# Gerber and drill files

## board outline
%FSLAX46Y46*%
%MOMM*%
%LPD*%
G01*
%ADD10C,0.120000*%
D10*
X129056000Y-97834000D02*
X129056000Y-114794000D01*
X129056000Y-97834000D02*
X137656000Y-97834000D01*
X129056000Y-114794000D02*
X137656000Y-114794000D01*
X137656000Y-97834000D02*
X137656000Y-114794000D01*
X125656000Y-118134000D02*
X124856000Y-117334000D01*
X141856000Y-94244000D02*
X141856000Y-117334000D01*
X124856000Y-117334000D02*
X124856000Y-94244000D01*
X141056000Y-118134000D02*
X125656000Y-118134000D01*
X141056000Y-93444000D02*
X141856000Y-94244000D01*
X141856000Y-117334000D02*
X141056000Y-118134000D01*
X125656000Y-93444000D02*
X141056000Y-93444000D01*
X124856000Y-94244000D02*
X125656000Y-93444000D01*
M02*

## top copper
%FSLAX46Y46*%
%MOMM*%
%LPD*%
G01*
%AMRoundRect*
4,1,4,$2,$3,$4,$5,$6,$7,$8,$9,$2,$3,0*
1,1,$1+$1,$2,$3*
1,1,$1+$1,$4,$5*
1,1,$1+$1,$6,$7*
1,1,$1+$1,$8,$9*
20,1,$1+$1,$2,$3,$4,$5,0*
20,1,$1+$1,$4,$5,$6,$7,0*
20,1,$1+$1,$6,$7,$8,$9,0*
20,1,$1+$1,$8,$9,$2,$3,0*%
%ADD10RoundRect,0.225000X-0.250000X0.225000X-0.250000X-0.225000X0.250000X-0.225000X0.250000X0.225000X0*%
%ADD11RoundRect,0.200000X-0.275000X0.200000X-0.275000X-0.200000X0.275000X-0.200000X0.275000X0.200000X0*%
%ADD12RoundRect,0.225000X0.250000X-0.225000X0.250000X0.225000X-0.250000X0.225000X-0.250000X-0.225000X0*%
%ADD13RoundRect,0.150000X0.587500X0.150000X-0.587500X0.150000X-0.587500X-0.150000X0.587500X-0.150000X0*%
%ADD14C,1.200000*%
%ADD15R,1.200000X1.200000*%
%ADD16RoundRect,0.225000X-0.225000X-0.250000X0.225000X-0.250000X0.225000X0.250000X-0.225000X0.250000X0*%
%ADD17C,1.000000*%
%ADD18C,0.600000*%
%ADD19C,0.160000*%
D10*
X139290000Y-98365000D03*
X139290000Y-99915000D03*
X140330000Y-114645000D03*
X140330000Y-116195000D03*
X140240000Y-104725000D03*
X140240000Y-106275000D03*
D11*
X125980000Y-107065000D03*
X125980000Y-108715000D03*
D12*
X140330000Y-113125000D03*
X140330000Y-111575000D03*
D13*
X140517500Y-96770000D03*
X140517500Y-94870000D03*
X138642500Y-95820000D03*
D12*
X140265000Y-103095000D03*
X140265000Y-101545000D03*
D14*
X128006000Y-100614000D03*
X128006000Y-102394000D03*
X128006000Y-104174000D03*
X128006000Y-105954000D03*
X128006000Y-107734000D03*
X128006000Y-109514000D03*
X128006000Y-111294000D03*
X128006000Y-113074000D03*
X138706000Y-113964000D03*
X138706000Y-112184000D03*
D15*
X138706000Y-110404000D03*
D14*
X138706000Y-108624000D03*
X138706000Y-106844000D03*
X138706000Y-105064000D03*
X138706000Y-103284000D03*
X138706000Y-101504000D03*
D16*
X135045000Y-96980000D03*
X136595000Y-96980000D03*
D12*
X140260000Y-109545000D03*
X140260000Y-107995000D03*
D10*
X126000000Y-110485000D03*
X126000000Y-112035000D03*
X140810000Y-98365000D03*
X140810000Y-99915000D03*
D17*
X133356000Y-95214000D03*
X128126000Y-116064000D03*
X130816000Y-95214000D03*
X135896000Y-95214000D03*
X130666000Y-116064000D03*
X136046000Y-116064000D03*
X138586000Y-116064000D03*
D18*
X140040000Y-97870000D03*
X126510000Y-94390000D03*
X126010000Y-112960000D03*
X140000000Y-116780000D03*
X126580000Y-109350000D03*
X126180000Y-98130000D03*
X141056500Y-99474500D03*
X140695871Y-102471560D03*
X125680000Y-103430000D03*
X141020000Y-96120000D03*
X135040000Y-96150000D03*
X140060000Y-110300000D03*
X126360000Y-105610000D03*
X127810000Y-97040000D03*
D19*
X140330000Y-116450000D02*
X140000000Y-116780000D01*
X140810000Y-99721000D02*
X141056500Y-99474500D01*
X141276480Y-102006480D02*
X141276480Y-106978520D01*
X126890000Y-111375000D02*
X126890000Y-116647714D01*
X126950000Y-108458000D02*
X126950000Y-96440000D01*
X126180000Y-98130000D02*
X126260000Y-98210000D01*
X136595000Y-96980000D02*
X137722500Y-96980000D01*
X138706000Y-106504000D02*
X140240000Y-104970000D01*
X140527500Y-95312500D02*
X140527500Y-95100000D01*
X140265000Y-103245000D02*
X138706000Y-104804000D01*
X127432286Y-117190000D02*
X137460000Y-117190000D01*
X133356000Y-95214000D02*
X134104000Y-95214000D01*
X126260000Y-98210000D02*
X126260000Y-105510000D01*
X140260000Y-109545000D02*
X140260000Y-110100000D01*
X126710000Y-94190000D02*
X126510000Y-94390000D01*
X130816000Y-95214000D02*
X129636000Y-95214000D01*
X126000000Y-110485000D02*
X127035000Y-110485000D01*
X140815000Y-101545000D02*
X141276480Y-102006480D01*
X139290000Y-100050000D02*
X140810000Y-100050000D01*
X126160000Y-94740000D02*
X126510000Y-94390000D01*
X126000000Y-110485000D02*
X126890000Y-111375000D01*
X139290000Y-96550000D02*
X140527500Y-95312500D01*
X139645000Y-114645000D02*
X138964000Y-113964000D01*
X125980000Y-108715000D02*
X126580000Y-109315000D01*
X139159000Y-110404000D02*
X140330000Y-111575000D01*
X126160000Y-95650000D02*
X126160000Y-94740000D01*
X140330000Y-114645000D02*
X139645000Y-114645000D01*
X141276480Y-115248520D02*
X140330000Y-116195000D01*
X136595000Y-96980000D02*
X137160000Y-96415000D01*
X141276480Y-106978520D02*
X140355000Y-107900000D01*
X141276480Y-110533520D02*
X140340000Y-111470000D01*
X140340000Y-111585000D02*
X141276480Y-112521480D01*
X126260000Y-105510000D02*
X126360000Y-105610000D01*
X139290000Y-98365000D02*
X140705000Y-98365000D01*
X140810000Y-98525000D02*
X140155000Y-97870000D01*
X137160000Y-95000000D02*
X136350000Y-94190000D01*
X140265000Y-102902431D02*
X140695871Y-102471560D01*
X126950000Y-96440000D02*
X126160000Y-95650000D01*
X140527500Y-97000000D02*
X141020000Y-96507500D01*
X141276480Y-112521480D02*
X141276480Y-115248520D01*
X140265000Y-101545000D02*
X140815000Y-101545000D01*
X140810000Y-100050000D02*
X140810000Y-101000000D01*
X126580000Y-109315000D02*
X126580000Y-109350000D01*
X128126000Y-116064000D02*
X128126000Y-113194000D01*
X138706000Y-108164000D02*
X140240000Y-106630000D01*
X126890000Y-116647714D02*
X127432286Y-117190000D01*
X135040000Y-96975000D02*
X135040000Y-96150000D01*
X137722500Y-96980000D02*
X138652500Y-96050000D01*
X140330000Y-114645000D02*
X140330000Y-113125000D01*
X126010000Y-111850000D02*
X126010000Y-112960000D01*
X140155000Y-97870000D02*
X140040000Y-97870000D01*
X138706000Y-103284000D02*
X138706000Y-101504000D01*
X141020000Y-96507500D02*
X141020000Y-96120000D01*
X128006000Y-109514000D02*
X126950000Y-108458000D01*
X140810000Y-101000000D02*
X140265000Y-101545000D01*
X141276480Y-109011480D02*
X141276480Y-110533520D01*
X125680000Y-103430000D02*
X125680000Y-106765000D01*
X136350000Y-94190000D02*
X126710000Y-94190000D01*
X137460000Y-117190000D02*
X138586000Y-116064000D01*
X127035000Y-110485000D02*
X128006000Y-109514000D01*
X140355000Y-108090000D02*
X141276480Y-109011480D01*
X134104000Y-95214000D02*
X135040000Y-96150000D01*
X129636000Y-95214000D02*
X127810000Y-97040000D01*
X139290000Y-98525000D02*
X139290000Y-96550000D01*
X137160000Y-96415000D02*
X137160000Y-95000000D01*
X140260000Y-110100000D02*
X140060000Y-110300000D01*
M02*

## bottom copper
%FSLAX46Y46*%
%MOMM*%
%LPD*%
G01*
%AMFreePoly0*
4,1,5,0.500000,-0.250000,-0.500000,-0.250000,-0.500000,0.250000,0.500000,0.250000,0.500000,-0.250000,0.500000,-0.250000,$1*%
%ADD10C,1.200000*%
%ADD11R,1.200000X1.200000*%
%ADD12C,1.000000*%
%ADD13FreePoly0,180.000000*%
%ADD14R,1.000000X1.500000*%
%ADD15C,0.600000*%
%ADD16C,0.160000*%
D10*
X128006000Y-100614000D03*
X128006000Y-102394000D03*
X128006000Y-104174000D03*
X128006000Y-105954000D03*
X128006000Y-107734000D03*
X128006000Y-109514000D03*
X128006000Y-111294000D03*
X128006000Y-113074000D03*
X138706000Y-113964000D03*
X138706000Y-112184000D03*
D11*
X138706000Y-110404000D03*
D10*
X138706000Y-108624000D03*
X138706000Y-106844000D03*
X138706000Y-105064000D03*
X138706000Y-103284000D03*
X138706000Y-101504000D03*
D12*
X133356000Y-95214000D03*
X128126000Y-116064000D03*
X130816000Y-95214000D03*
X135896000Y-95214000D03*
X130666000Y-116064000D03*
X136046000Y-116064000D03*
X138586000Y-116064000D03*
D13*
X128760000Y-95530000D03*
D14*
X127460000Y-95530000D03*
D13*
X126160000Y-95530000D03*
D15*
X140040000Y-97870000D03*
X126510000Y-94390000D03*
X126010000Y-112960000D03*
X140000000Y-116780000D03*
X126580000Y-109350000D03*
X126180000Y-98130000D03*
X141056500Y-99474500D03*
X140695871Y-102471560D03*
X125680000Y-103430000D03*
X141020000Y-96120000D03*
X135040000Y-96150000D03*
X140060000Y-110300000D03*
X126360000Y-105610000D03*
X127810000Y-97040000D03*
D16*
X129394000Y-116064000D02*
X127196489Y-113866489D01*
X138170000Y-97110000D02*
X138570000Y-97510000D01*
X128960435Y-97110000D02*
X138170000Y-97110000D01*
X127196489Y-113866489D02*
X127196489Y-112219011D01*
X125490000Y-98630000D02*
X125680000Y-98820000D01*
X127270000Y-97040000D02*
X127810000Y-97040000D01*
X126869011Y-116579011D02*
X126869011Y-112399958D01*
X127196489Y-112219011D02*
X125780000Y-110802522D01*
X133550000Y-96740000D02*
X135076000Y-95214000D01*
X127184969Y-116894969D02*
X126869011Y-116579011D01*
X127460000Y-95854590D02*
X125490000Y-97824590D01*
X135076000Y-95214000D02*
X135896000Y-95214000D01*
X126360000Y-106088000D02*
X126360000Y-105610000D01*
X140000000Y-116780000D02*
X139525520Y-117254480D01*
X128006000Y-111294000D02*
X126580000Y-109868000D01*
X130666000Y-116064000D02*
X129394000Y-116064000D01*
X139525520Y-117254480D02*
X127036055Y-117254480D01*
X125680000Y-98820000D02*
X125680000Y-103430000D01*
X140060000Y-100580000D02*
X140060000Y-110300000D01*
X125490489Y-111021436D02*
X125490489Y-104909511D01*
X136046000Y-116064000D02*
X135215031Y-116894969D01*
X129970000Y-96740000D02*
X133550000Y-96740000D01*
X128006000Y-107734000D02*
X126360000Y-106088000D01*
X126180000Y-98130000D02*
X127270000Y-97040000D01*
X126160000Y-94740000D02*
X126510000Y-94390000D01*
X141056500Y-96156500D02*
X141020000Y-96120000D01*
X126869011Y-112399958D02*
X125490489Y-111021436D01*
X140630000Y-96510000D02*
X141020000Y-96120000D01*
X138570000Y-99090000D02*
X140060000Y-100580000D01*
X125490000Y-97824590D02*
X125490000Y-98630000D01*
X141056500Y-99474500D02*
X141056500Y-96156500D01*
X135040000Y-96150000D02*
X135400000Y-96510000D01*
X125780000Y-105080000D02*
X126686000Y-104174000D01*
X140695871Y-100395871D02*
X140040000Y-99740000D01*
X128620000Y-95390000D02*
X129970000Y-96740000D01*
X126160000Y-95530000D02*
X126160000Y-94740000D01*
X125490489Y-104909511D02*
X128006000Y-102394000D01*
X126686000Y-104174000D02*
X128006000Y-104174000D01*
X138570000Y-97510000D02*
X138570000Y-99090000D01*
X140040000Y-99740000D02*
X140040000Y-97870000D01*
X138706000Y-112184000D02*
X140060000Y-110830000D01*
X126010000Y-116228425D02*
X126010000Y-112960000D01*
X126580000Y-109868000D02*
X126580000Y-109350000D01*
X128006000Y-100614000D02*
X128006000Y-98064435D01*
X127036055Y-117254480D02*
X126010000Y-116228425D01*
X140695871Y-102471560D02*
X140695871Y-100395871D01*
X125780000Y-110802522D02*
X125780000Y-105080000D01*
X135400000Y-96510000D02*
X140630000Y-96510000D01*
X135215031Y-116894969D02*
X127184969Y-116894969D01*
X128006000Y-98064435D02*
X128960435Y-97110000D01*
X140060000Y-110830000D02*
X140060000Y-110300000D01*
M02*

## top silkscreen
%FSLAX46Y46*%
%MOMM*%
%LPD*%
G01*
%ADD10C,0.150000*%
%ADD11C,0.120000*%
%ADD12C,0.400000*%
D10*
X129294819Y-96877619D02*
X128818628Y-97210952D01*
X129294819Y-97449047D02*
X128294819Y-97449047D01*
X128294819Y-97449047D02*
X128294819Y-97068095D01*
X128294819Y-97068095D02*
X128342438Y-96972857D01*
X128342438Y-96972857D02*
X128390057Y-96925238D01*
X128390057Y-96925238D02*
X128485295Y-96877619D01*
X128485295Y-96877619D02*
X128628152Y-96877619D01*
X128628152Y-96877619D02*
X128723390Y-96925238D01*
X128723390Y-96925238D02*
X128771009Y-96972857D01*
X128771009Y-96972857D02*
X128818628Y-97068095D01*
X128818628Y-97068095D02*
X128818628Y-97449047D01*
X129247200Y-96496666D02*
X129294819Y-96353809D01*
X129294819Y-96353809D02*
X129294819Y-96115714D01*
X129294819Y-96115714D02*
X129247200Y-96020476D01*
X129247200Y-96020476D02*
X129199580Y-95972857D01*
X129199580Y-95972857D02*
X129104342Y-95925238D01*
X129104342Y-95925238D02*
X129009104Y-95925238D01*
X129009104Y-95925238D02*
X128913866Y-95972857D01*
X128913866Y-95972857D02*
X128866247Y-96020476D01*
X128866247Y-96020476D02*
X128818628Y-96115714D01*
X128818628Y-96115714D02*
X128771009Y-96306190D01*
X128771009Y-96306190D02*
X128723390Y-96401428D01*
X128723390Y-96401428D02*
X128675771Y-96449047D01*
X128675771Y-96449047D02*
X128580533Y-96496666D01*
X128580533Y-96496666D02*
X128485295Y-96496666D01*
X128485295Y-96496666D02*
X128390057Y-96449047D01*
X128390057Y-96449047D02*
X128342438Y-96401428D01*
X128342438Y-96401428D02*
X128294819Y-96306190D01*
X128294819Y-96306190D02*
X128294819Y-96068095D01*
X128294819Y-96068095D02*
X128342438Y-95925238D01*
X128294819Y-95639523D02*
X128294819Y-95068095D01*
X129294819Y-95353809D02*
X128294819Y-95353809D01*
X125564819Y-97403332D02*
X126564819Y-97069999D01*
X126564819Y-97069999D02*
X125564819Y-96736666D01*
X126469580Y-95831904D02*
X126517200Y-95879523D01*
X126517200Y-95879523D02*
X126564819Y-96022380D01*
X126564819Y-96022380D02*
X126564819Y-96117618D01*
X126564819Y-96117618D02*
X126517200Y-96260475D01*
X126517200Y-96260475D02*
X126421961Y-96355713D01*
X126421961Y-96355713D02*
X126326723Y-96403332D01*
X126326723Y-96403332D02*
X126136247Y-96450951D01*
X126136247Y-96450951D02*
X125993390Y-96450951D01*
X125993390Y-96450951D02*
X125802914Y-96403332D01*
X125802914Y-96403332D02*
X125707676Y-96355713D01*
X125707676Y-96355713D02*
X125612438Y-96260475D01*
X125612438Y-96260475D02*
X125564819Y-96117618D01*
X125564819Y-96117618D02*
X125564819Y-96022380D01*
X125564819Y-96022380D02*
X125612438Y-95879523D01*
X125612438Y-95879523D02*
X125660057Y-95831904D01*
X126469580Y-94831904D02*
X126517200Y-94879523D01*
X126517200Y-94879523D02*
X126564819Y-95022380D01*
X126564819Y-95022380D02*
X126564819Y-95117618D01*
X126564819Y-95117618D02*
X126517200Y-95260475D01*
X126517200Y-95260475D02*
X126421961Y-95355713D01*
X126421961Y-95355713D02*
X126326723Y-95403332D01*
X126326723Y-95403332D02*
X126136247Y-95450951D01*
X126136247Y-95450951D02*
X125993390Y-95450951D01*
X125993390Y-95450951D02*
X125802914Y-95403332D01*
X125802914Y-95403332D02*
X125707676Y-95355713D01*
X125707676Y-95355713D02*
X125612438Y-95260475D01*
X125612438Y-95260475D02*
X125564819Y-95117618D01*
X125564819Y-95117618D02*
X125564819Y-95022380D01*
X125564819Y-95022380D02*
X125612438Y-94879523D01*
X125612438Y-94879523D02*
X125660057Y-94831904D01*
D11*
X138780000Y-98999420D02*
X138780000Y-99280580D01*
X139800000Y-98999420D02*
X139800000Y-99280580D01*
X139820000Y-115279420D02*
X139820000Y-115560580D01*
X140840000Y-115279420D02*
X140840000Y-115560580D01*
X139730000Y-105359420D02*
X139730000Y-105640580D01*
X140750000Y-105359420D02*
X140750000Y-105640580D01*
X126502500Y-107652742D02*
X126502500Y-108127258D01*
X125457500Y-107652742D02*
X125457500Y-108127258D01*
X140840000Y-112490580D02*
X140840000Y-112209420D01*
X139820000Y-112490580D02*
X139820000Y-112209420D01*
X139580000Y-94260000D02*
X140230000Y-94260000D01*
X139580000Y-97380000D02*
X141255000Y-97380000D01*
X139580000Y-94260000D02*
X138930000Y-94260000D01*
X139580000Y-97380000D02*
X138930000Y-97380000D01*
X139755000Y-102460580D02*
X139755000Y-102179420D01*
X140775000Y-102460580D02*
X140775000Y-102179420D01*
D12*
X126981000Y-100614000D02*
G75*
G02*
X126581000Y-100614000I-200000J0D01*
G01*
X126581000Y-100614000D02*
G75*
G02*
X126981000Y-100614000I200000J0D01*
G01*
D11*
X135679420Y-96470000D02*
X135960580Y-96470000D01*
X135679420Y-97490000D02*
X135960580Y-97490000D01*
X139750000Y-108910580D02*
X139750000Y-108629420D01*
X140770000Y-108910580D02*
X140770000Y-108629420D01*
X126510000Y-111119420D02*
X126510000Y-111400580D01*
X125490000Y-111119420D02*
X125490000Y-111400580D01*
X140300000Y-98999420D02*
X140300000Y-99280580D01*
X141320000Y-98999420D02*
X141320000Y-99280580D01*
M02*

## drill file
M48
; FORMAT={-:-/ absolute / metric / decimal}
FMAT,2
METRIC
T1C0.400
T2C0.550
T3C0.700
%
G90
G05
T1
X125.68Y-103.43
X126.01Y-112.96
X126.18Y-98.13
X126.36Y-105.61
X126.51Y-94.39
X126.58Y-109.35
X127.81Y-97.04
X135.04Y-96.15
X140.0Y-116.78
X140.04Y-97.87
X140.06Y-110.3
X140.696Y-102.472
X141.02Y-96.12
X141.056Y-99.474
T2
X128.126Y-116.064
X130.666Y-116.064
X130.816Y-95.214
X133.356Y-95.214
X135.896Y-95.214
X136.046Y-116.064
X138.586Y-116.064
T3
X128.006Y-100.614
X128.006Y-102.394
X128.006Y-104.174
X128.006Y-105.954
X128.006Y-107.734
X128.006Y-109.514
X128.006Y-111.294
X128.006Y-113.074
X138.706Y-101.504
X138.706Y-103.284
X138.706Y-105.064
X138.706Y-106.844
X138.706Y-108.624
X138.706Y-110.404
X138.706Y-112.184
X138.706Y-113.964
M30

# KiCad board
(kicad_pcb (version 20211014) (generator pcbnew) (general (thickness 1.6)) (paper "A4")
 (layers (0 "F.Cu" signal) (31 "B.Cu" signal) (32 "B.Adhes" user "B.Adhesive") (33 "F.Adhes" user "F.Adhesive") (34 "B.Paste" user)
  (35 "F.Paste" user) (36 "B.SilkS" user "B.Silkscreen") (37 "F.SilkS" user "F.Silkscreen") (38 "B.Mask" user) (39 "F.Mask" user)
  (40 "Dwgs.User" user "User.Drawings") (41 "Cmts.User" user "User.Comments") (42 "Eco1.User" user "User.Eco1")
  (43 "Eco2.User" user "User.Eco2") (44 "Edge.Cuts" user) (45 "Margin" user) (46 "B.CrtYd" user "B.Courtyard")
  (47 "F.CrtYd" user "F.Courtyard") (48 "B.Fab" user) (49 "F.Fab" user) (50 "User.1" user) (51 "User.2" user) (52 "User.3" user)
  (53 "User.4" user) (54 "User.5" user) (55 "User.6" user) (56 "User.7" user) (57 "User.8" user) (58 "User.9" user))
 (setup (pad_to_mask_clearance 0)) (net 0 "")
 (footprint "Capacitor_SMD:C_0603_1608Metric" (layer "F.Cu") (at 139.29 99.14 -90)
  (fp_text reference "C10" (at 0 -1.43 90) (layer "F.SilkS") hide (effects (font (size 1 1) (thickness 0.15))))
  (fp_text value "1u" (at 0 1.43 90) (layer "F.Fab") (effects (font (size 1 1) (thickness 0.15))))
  (fp_line (start -0.14058 0.51) (end 0.14058 0.51) (layer "F.SilkS") (width 0.12))
  (fp_line (start -0.14058 -0.51) (end 0.14058 -0.51) (layer "F.SilkS") (width 0.12))
  (pad "1" smd roundrect (at -0.775 0 270) (size 0.9 0.95) (layers "F.Cu" "F.Paste" "F.Mask") (roundrect_rratio 0.25))
  (pad "2" smd roundrect (at 0.775 0 270) (size 0.9 0.95) (layers "F.Cu" "F.Paste" "F.Mask") (roundrect_rratio 0.25)))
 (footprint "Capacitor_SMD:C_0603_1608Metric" (layer "F.Cu") (at 140.33 115.42 -90)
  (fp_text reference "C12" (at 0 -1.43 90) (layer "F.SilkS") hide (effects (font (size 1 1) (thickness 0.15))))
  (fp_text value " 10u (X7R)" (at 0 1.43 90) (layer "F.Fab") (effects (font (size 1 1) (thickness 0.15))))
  (fp_line (start -0.14058 0.51) (end 0.14058 0.51) (layer "F.SilkS") (width 0.12))
  (fp_line (start -0.14058 -0.51) (end 0.14058 -0.51) (layer "F.SilkS") (width 0.12))
  (pad "1" smd roundrect (at -0.775 0 270) (size 0.9 0.95) (layers "F.Cu" "F.Paste" "F.Mask") (roundrect_rratio 0.25))
  (pad "2" smd roundrect (at 0.775 0 270) (size 0.9 0.95) (layers "F.Cu" "F.Paste" "F.Mask") (roundrect_rratio 0.25)))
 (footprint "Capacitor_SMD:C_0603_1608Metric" (layer "F.Cu") (at 140.24 105.5 -90)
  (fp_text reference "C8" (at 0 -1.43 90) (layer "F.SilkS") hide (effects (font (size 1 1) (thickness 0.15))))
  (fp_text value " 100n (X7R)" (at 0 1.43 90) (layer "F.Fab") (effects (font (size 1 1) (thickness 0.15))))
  (fp_line (start -0.14058 0.51) (end 0.14058 0.51) (layer "F.SilkS") (width 0.12))
  (fp_line (start -0.14058 -0.51) (end 0.14058 -0.51) (layer "F.SilkS") (width 0.12))
  (pad "1" smd roundrect (at -0.775 0 270) (size 0.9 0.95) (layers "F.Cu" "F.Paste" "F.Mask") (roundrect_rratio 0.25))
  (pad "2" smd roundrect (at 0.775 0 270) (size 0.9 0.95) (layers "F.Cu" "F.Paste" "F.Mask") (roundrect_rratio 0.25)))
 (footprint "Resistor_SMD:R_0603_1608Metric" (layer "F.Cu") (at 125.98 107.89 -90)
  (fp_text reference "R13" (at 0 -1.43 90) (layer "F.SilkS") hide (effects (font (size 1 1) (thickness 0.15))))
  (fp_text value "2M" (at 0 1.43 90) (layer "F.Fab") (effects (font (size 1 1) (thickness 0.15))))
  (fp_line (start -0.237258 -0.5225) (end 0.237258 -0.5225) (layer "F.SilkS") (width 0.12))
  (fp_line (start -0.237258 0.5225) (end 0.237258 0.5225) (layer "F.SilkS") (width 0.12))
  (pad "1" smd roundrect (at -0.825 0 270) (size 0.8 0.95) (layers "F.Cu" "F.Paste" "F.Mask") (roundrect_rratio 0.25))
  (pad "2" smd roundrect (at 0.825 0 270) (size 0.8 0.95) (layers "F.Cu" "F.Paste" "F.Mask") (roundrect_rratio 0.25)))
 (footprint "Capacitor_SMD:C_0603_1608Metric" (layer "F.Cu") (at 140.33 112.35 90)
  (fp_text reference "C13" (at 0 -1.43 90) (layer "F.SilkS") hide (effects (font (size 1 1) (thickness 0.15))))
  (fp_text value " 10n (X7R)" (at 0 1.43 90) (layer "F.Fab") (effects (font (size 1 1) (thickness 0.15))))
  (fp_line (start -0.14058 0.51) (end 0.14058 0.51) (layer "F.SilkS") (width 0.12))
  (fp_line (start -0.14058 -0.51) (end 0.14058 -0.51) (layer "F.SilkS") (width 0.12))
  (pad "1" smd roundrect (at -0.775 0 90) (size 0.9 0.95) (layers "F.Cu" "F.Paste" "F.Mask") (roundrect_rratio 0.25))
  (pad "2" smd roundrect (at 0.775 0 90) (size 0.9 0.95) (layers "F.Cu" "F.Paste" "F.Mask") (roundrect_rratio 0.25)))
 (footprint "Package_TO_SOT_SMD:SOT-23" (layer "F.Cu") (at 139.58 95.82 180)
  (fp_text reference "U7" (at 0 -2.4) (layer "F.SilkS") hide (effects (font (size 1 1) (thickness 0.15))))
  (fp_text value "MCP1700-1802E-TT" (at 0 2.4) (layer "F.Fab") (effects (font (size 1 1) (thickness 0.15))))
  (fp_line (start 0 1.56) (end -0.65 1.56) (layer "F.SilkS") (width 0.12))
  (fp_line (start 0 -1.56) (end -1.675 -1.56) (layer "F.SilkS") (width 0.12))
  (fp_line (start 0 1.56) (end 0.65 1.56) (layer "F.SilkS") (width 0.12))
  (fp_line (start 0 -1.56) (end 0.65 -1.56) (layer "F.SilkS") (width 0.12))
  (pad "1" smd roundrect (at -0.9375 -0.95 180) (size 1.475 0.6) (layers "F.Cu" "F.Paste" "F.Mask") (roundrect_rratio 0.25))
  (pad "2" smd roundrect (at -0.9375 0.95 180) (size 1.475 0.6) (layers "F.Cu" "F.Paste" "F.Mask") (roundrect_rratio 0.25))
  (pad "3" smd roundrect (at 0.9375 0 180) (size 1.475 0.6) (layers "F.Cu" "F.Paste" "F.Mask") (roundrect_rratio 0.25)))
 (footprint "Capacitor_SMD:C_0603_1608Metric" (layer "F.Cu") (at 140.265 102.32 90)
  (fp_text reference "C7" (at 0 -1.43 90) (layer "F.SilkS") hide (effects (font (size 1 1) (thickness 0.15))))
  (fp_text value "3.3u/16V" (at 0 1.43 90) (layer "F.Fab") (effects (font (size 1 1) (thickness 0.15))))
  (fp_line (start -0.14058 -0.51) (end 0.14058 -0.51) (layer "F.SilkS") (width 0.12))
  (fp_line (start -0.14058 0.51) (end 0.14058 0.51) (layer "F.SilkS") (width 0.12))
  (pad "1" smd roundrect (at -0.775 0 90) (size 0.9 0.95) (layers "F.Cu" "F.Paste" "F.Mask") (roundrect_rratio 0.25))
  (pad "2" smd roundrect (at 0.775 0 90) (size 0.9 0.95) (layers "F.Cu" "F.Paste" "F.Mask") (roundrect_rratio 0.25)))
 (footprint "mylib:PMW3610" (layer "F.Cu") (at 128.006 100.614)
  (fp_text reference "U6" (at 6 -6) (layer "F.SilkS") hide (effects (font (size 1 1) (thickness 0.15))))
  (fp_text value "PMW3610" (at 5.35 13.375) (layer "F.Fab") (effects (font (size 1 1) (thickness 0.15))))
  (fp_circle (center -1.225 0) (end -1.025 0) (layer "F.SilkS") (width 0.4) (fill none))
  (fp_line (start 1.05 -2.78) (end 1.05 14.18) (layer "Edge.Cuts") (width 0.12))
  (fp_line (start 1.05 -2.78) (end 9.65 -2.78) (layer "Edge.Cuts") (width 0.12))
  (fp_line (start 1.05 14.18) (end 9.65 14.18) (layer "Edge.Cuts") (width 0.12))
  (fp_line (start 9.65 -2.78) (end 9.65 14.18) (layer "Edge.Cuts") (width 0.12))
  (pad "1" thru_hole circle (at 0 0) (size 1.2 1.2) (drill 0.7) (layers *.Cu *.Mask))
  (pad "2" thru_hole circle (at 0 1.78) (size 1.2 1.2) (drill 0.7) (layers *.Cu *.Mask))
  (pad "3" thru_hole circle (at 0 3.56) (size 1.2 1.2) (drill 0.7) (layers *.Cu *.Mask))
  (pad "4" thru_hole circle (at 0 5.34) (size 1.2 1.2) (drill 0.7) (layers *.Cu *.Mask))
  (pad "5" thru_hole circle (at 0 7.12) (size 1.2 1.2) (drill 0.7) (layers *.Cu *.Mask))
  (pad "6" thru_hole circle (at 0 8.9) (size 1.2 1.2) (drill 0.7) (layers *.Cu *.Mask))
  (pad "7" thru_hole circle (at 0 10.68) (size 1.2 1.2) (drill 0.7) (layers *.Cu *.Mask))
  (pad "8" thru_hole circle (at 0 12.46) (size 1.2 1.2) (drill 0.7) (layers *.Cu *.Mask))
  (pad "9" thru_hole circle (at 10.7 13.35) (size 1.2 1.2) (drill 0.7) (layers *.Cu *.Mask))
  (pad "10" thru_hole circle (at 10.7 11.57) (size 1.2 1.2) (drill 0.7) (layers *.Cu *.Mask))
  (pad "11" thru_hole rect (at 10.7 9.79) (size 1.2 1.2) (drill 0.7) (layers *.Cu *.Mask))
  (pad "12" thru_hole circle (at 10.7 8.01) (size 1.2 1.2) (drill 0.7) (layers *.Cu *.Mask))
  (pad "13" thru_hole circle (at 10.7 6.23) (size 1.2 1.2) (drill 0.7) (layers *.Cu *.Mask))
  (pad "14" thru_hole circle (at 10.7 4.45) (size 1.2 1.2) (drill 0.7) (layers *.Cu *.Mask))
  (pad "15" thru_hole circle (at 10.7 2.67) (size 1.2 1.2) (drill 0.7) (layers *.Cu *.Mask))
  (pad "16" thru_hole circle (at 10.7 0.89) (size 1.2 1.2) (drill 0.7) (layers *.Cu *.Mask)))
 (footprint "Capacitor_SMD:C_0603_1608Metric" (layer "F.Cu") (at 135.82 96.98)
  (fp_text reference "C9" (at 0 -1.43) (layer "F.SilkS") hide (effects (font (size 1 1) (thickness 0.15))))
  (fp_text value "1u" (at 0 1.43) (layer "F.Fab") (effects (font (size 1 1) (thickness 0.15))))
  (fp_line (start -0.14058 -0.51) (end 0.14058 -0.51) (layer "F.SilkS") (width 0.12))
  (fp_line (start -0.14058 0.51) (end 0.14058 0.51) (layer "F.SilkS") (width 0.12))
  (pad "1" smd roundrect (at -0.775 0) (size 0.9 0.95) (layers "F.Cu" "F.Paste" "F.Mask") (roundrect_rratio 0.25))
  (pad "2" smd roundrect (at 0.775 0) (size 0.9 0.95) (layers "F.Cu" "F.Paste" "F.Mask") (roundrect_rratio 0.25)))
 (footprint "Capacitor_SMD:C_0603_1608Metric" (layer "F.Cu") (at 140.26 108.77 90)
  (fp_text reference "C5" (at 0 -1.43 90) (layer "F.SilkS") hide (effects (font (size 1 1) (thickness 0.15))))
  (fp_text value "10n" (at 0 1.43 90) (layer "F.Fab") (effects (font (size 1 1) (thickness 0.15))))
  (fp_line (start -0.14058 -0.51) (end 0.14058 -0.51) (layer "F.SilkS") (width 0.12))
  (fp_line (start -0.14058 0.51) (end 0.14058 0.51) (layer "F.SilkS") (width 0.12))
  (pad "1" smd roundrect (at -0.775 0 90) (size 0.9 0.95) (layers "F.Cu" "F.Paste" "F.Mask") (roundrect_rratio 0.25))
  (pad "2" smd roundrect (at 0.775 0 90) (size 0.9 0.95) (layers "F.Cu" "F.Paste" "F.Mask") (roundrect_rratio 0.25)))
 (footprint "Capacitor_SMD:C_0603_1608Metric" (layer "F.Cu") (at 126 111.26 -90)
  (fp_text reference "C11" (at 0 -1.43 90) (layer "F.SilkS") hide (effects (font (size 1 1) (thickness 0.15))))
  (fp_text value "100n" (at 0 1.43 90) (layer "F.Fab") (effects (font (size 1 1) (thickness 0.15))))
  (fp_line (start -0.14058 -0.51) (end 0.14058 -0.51) (layer "F.SilkS") (width 0.12))
  (fp_line (start -0.14058 0.51) (end 0.14058 0.51) (layer "F.SilkS") (width 0.12))
  (pad "1" smd roundrect (at -0.775 0 270) (size 0.9 0.95) (layers "F.Cu" "F.Paste" "F.Mask") (roundrect_rratio 0.25))
  (pad "2" smd roundrect (at 0.775 0 270) (size 0.9 0.95) (layers "F.Cu" "F.Paste" "F.Mask") (roundrect_rratio 0.25)))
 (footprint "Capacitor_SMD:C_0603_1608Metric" (layer "F.Cu") (at 140.81 99.14 -90)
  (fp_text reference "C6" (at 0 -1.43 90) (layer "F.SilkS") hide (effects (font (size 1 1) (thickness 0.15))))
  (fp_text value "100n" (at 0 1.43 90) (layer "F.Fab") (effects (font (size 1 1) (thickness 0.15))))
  (fp_line (start -0.14058 0.51) (end 0.14058 0.51) (layer "F.SilkS") (width 0.12))
  (fp_line (start -0.14058 -0.51) (end 0.14058 -0.51) (layer "F.SilkS") (width 0.12))
  (pad "1" smd roundrect (at -0.775 0 270) (size 0.9 0.95) (layers "F.Cu" "F.Paste" "F.Mask") (roundrect_rratio 0.25))
  (pad "2" smd roundrect (at 0.775 0 270) (size 0.9 0.95) (layers "F.Cu" "F.Paste" "F.Mask") (roundrect_rratio 0.25)))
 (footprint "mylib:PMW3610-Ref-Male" (layer "F.Cu") (at 128.006 100.614)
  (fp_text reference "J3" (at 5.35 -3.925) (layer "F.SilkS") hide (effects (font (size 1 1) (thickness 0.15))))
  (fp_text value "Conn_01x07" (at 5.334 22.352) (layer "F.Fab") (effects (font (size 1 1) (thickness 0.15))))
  (fp_line (start -2.35 17.52) (end -3.15 16.72) (layer "Edge.Cuts") (width 0.12))
  (fp_line (start 13.85 -6.37) (end 13.85 16.72) (layer "Edge.Cuts") (width 0.12))
  (fp_line (start -3.15 16.72) (end -3.15 -6.37) (layer "Edge.Cuts") (width 0.12))
  (fp_line (start 13.05 17.52) (end -2.35 17.52) (layer "Edge.Cuts") (width 0.12))
  (fp_line (start 13.05 -7.17) (end 13.85 -6.37) (layer "Edge.Cuts") (width 0.12))
  (fp_line (start 13.85 16.72) (end 13.05 17.52) (layer "Edge.Cuts") (width 0.12))
  (fp_line (start -2.35 -7.17) (end 13.05 -7.17) (layer "Edge.Cuts") (width 0.12))
  (fp_line (start -3.15 -6.37) (end -2.35 -7.17) (layer "Edge.Cuts") (width 0.12))
  (pad "gnd" thru_hole circle (at 5.35 -5.4) (size 1 1) (drill 0.55) (layers *.Cu *.Mask))
  (pad "intr" thru_hole circle (at 0.12 15.45) (size 1 1) (drill 0.55) (layers *.Cu *.Mask))
  (pad "ncs" thru_hole circle (at 2.81 -5.4) (size 1 1) (drill 0.55) (layers *.Cu *.Mask))
  (pad "rst" thru_hole circle (at 7.89 -5.4) (size 1 1) (drill 0.55) (layers *.Cu *.Mask))
  (pad "sclk" thru_hole circle (at 2.66 15.45) (size 1 1) (drill 0.55) (layers *.Cu *.Mask))
  (pad "sdio" thru_hole circle (at 8.04 15.45) (size 1 1) (drill 0.55) (layers *.Cu *.Mask))
  (pad "vcc" thru_hole circle (at 10.58 15.45) (size 1 1) (drill 0.55) (layers *.Cu *.Mask)))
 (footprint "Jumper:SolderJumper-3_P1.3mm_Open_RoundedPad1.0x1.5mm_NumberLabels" (layer "B.Cu") (at 127.46 95.53 180)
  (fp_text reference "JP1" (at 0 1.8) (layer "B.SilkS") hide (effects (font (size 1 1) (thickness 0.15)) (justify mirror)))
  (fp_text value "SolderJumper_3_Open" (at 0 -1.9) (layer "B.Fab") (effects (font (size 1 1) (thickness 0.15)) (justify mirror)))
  (pad "1" smd custom (at -1.3 0 180) (size 1 0.5) (layers "B.Cu" "B.Mask") (zone_connect 2) (options (clearance outline) (anchor rect))
   (primitives))
  (pad "2" smd rect (at 0 0 180) (size 1 1.5) (layers "B.Cu" "B.Mask"))
  (pad "3" smd custom (at 1.3 0 180) (size 1 0.5) (layers "B.Cu" "B.Mask") (zone_connect 2) (options (clearance outline) (anchor rect))
   (primitives)))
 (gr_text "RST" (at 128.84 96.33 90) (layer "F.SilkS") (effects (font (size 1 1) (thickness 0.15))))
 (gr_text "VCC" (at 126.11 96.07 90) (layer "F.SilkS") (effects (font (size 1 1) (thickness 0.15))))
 (segment (start 140.33 116.45) (end 140 116.78) (width 0.16) (layer "F.Cu") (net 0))
 (segment (start 140.81 99.721) (end 141.0565 99.4745) (width 0.16) (layer "F.Cu") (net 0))
 (segment (start 141.27648 102.00648) (end 141.27648 106.97852) (width 0.16) (layer "F.Cu") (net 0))
 (segment (start 126.89 111.375) (end 126.89 116.647714) (width 0.16) (layer "F.Cu") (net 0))
 (segment (start 126.95 108.458) (end 126.95 96.44) (width 0.16) (layer "F.Cu") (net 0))
 (segment (start 126.18 98.13) (end 126.26 98.21) (width 0.16) (layer "F.Cu") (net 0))
 (segment (start 136.595 96.98) (end 137.7225 96.98) (width 0.16) (layer "F.Cu") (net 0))
 (segment (start 138.706 106.504) (end 140.24 104.97) (width 0.16) (layer "F.Cu") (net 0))
 (segment (start 140.5275 95.3125) (end 140.5275 95.1) (width 0.16) (layer "F.Cu") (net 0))
 (segment (start 140.265 103.245) (end 138.706 104.804) (width 0.16) (layer "F.Cu") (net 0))
 (segment (start 127.432286 117.19) (end 137.46 117.19) (width 0.16) (layer "F.Cu") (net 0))
 (segment (start 133.356 95.214) (end 134.104 95.214) (width 0.16) (layer "F.Cu") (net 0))
 (segment (start 126.26 98.21) (end 126.26 105.51) (width 0.16) (layer "F.Cu") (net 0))
 (segment (start 140.26 109.545) (end 140.26 110.1) (width 0.16) (layer "F.Cu") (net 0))
 (segment (start 126.71 94.19) (end 126.51 94.39) (width 0.16) (layer "F.Cu") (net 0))
 (segment (start 130.816 95.214) (end 129.636 95.214) (width 0.16) (layer "F.Cu") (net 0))
 (segment (start 126 110.485) (end 127.035 110.485) (width 0.16) (layer "F.Cu") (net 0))
 (segment (start 140.815 101.545) (end 141.27648 102.00648) (width 0.16) (layer "F.Cu") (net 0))
 (segment (start 139.29 100.05) (end 140.81 100.05) (width 0.16) (layer "F.Cu") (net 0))
 (segment (start 126.16 94.74) (end 126.51 94.39) (width 0.16) (layer "F.Cu") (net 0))
 (segment (start 126 110.485) (end 126.89 111.375) (width 0.16) (layer "F.Cu") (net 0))
 (segment (start 139.29 96.55) (end 140.5275 95.3125) (width 0.16) (layer "F.Cu") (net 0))
 (segment (start 139.645 114.645) (end 138.964 113.964) (width 0.16) (layer "F.Cu") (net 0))
 (segment (start 125.98 108.715) (end 126.58 109.315) (width 0.16) (layer "F.Cu") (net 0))
 (segment (start 139.159 110.404) (end 140.33 111.575) (width 0.16) (layer "F.Cu") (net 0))
 (segment (start 126.16 95.65) (end 126.16 94.74) (width 0.16) (layer "F.Cu") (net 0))
 (segment (start 140.33 114.645) (end 139.645 114.645) (width 0.16) (layer "F.Cu") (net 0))
 (segment (start 141.27648 115.24852) (end 140.33 116.195) (width 0.16) (layer "F.Cu") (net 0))
 (segment (start 136.595 96.98) (end 137.16 96.415) (width 0.16) (layer "F.Cu") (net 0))
 (segment (start 141.27648 106.97852) (end 140.355 107.9) (width 0.16) (layer "F.Cu") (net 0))
 (segment (start 141.27648 110.53352) (end 140.34 111.47) (width 0.16) (layer "F.Cu") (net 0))
 (segment (start 140.34 111.585) (end 141.27648 112.52148) (width 0.16) (layer "F.Cu") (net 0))
 (segment (start 126.26 105.51) (end 126.36 105.61) (width 0.16) (layer "F.Cu") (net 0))
 (segment (start 139.29 98.365) (end 140.705 98.365) (width 0.16) (layer "F.Cu") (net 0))
 (segment (start 140.81 98.525) (end 140.155 97.87) (width 0.16) (layer "F.Cu") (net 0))
 (segment (start 137.16 95) (end 136.35 94.19) (width 0.16) (layer "F.Cu") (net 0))
 (segment (start 140.265 102.902431) (end 140.695871 102.47156) (width 0.16) (layer "F.Cu") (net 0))
 (segment (start 126.95 96.44) (end 126.16 95.65) (width 0.16) (layer "F.Cu") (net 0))
 (segment (start 140.5275 97) (end 141.02 96.5075) (width 0.16) (layer "F.Cu") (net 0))
 (segment (start 141.27648 112.52148) (end 141.27648 115.24852) (width 0.16) (layer "F.Cu") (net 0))
 (segment (start 140.265 101.545) (end 140.815 101.545) (width 0.16) (layer "F.Cu") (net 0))
 (segment (start 140.81 100.05) (end 140.81 101) (width 0.16) (layer "F.Cu") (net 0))
 (segment (start 126.58 109.315) (end 126.58 109.35) (width 0.16) (layer "F.Cu") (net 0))
 (segment (start 128.126 116.064) (end 128.126 113.194) (width 0.16) (layer "F.Cu") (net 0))
 (segment (start 138.706 108.164) (end 140.24 106.63) (width 0.16) (layer "F.Cu") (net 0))
 (segment (start 126.89 116.647714) (end 127.432286 117.19) (width 0.16) (layer "F.Cu") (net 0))
 (segment (start 135.04 96.975) (end 135.04 96.15) (width 0.16) (layer "F.Cu") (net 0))
 (segment (start 137.7225 96.98) (end 138.6525 96.05) (width 0.16) (layer "F.Cu") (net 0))
 (segment (start 140.33 114.645) (end 140.33 113.125) (width 0.16) (layer "F.Cu") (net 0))
 (segment (start 126.01 111.85) (end 126.01 112.96) (width 0.16) (layer "F.Cu") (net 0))
 (segment (start 140.155 97.87) (end 140.04 97.87) (width 0.16) (layer "F.Cu") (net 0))
 (segment (start 138.706 103.284) (end 138.706 101.504) (width 0.16) (layer "F.Cu") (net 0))
 (segment (start 141.02 96.5075) (end 141.02 96.12) (width 0.16) (layer "F.Cu") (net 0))
 (segment (start 128.006 109.514) (end 126.95 108.458) (width 0.16) (layer "F.Cu") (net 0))
 (segment (start 140.81 101) (end 140.265 101.545) (width 0.16) (layer "F.Cu") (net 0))
 (segment (start 141.27648 109.01148) (end 141.27648 110.53352) (width 0.16) (layer "F.Cu") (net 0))
 (segment (start 125.68 103.43) (end 125.68 106.765) (width 0.16) (layer "F.Cu") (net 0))
 (segment (start 136.35 94.19) (end 126.71 94.19) (width 0.16) (layer "F.Cu") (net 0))
 (segment (start 137.46 117.19) (end 138.586 116.064) (width 0.16) (layer "F.Cu") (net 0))
 (segment (start 127.035 110.485) (end 128.006 109.514) (width 0.16) (layer "F.Cu") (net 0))
 (segment (start 140.355 108.09) (end 141.27648 109.01148) (width 0.16) (layer "F.Cu") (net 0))
 (segment (start 134.104 95.214) (end 135.04 96.15) (width 0.16) (layer "F.Cu") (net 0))
 (segment (start 129.636 95.214) (end 127.81 97.04) (width 0.16) (layer "F.Cu") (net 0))
 (segment (start 139.29 98.525) (end 139.29 96.55) (width 0.16) (layer "F.Cu") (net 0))
 (segment (start 137.16 96.415) (end 137.16 95) (width 0.16) (layer "F.Cu") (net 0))
 (segment (start 140.26 110.1) (end 140.06 110.3) (width 0.16) (layer "F.Cu") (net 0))
 (via (at 140.04 97.87) (size 0.6) (drill 0.4) (layers "F.Cu" "B.Cu") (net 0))
 (via (at 126.51 94.39) (size 0.6) (drill 0.4) (layers "F.Cu" "B.Cu") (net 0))
 (via (at 126.01 112.96) (size 0.6) (drill 0.4) (layers "F.Cu" "B.Cu") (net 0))
 (via (at 140 116.78) (size 0.6) (drill 0.4) (layers "F.Cu" "B.Cu") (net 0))
 (via (at 126.58 109.35) (size 0.6) (drill 0.4) (layers "F.Cu" "B.Cu") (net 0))
 (via (at 126.18 98.13) (size 0.6) (drill 0.4) (layers "F.Cu" "B.Cu") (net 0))
 (via (at 141.0565 99.4745) (size 0.6) (drill 0.4) (layers "F.Cu" "B.Cu") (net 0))
 (via (at 140.695871 102.47156) (size 0.6) (drill 0.4) (layers "F.Cu" "B.Cu") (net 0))
 (via (at 125.68 103.43) (size 0.6) (drill 0.4) (layers "F.Cu" "B.Cu") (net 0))
 (via (at 141.02 96.12) (size 0.6) (drill 0.4) (layers "F.Cu" "B.Cu") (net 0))
 (via (at 135.04 96.15) (size 0.6) (drill 0.4) (layers "F.Cu" "B.Cu") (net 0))
 (via (at 140.06 110.3) (size 0.6) (drill 0.4) (layers "F.Cu" "B.Cu") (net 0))
 (via (at 126.36 105.61) (size 0.6) (drill 0.4) (layers "F.Cu" "B.Cu") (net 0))
 (via (at 127.81 97.04) (size 0.6) (drill 0.4) (layers "F.Cu" "B.Cu") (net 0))
 (segment (start 129.394 116.064) (end 127.196489 113.866489) (width 0.16) (layer "B.Cu") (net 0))
 (segment (start 138.17 97.11) (end 138.57 97.51) (width 0.16) (layer "B.Cu") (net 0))
 (segment (start 128.960435 97.11) (end 138.17 97.11) (width 0.16) (layer "B.Cu") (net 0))
 (segment (start 127.196489 113.866489) (end 127.196489 112.219011) (width 0.16) (layer "B.Cu") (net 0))
 (segment (start 125.49 98.63) (end 125.68 98.82) (width 0.16) (layer "B.Cu") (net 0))
 (segment (start 127.27 97.04) (end 127.81 97.04) (width 0.16) (layer "B.Cu") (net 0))
 (segment (start 126.869011 116.579011) (end 126.869011 112.399958) (width 0.16) (layer "B.Cu") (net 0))
 (segment (start 127.196489 112.219011) (end 125.78 110.802522) (width 0.16) (layer "B.Cu") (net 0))
 (segment (start 133.55 96.74) (end 135.076 95.214) (width 0.16) (layer "B.Cu") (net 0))
 (segment (start 127.184969 116.894969) (end 126.869011 116.579011) (width 0.16) (layer "B.Cu") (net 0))
 (segment (start 127.46 95.85459) (end 125.49 97.82459) (width 0.16) (layer "B.Cu") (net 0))
 (segment (start 135.076 95.214) (end 135.896 95.214) (width 0.16) (layer "B.Cu") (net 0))
 (segment (start 126.36 106.088) (end 126.36 105.61) (width 0.16) (layer "B.Cu") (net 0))
 (segment (start 140 116.78) (end 139.52552 117.25448) (width 0.16) (layer "B.Cu") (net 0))
 (segment (start 128.006 111.294) (end 126.58 109.868) (width 0.16) (layer "B.Cu") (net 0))
 (segment (start 130.666 116.064) (end 129.394 116.064) (width 0.16) (layer "B.Cu") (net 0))
 (segment (start 139.52552 117.25448) (end 127.036055 117.25448) (width 0.16) (layer "B.Cu") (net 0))
 (segment (start 125.68 98.82) (end 125.68 103.43) (width 0.16) (layer "B.Cu") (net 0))
 (segment (start 140.06 100.58) (end 140.06 110.3) (width 0.16) (layer "B.Cu") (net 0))
 (segment (start 125.490489 111.021436) (end 125.490489 104.909511) (width 0.16) (layer "B.Cu") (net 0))
 (segment (start 136.046 116.064) (end 135.215031 116.894969) (width 0.16) (layer "B.Cu") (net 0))
 (segment (start 129.97 96.74) (end 133.55 96.74) (width 0.16) (layer "B.Cu") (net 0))
 (segment (start 128.006 107.734) (end 126.36 106.088) (width 0.16) (layer "B.Cu") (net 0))
 (segment (start 126.18 98.13) (end 127.27 97.04) (width 0.16) (layer "B.Cu") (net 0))
 (segment (start 126.16 94.74) (end 126.51 94.39) (width 0.16) (layer "B.Cu") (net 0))
 (segment (start 141.0565 96.1565) (end 141.02 96.12) (width 0.16) (layer "B.Cu") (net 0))
 (segment (start 126.869011 112.399958) (end 125.490489 111.021436) (width 0.16) (layer "B.Cu") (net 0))
 (segment (start 140.63 96.51) (end 141.02 96.12) (width 0.16) (layer "B.Cu") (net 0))
 (segment (start 138.57 99.09) (end 140.06 100.58) (width 0.16) (layer "B.Cu") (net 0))
 (segment (start 125.49 97.82459) (end 125.49 98.63) (width 0.16) (layer "B.Cu") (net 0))
 (segment (start 141.0565 99.4745) (end 141.0565 96.1565) (width 0.16) (layer "B.Cu") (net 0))
 (segment (start 135.04 96.15) (end 135.4 96.51) (width 0.16) (layer "B.Cu") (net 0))
 (segment (start 125.78 105.08) (end 126.686 104.174) (width 0.16) (layer "B.Cu") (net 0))
 (segment (start 140.695871 100.395871) (end 140.04 99.74) (width 0.16) (layer "B.Cu") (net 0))
 (segment (start 128.62 95.39) (end 129.97 96.74) (width 0.16) (layer "B.Cu") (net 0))
 (segment (start 126.16 95.53) (end 126.16 94.74) (width 0.16) (layer "B.Cu") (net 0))
 (segment (start 125.490489 104.909511) (end 128.006 102.394) (width 0.16) (layer "B.Cu") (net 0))
 (segment (start 126.686 104.174) (end 128.006 104.174) (width 0.16) (layer "B.Cu") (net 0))
 (segment (start 138.57 97.51) (end 138.57 99.09) (width 0.16) (layer "B.Cu") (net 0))
 (segment (start 140.04 99.74) (end 140.04 97.87) (width 0.16) (layer "B.Cu") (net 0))
 (segment (start 138.706 112.184) (end 140.06 110.83) (width 0.16) (layer "B.Cu") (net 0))
 (segment (start 126.01 116.228425) (end 126.01 112.96) (width 0.16) (layer "B.Cu") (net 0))
 (segment (start 126.58 109.868) (end 126.58 109.35) (width 0.16) (layer "B.Cu") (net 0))
 (segment (start 128.006 100.614) (end 128.006 98.064435) (width 0.16) (layer "B.Cu") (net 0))
 (segment (start 127.036055 117.25448) (end 126.01 116.228425) (width 0.16) (layer "B.Cu") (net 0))
 (segment (start 140.695871 102.47156) (end 140.695871 100.395871) (width 0.16) (layer "B.Cu") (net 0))
 (segment (start 125.78 110.802522) (end 125.78 105.08) (width 0.16) (layer "B.Cu") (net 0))
 (segment (start 135.4 96.51) (end 140.63 96.51) (width 0.16) (layer "B.Cu") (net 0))
 (segment (start 135.215031 116.894969) (end 127.184969 116.894969) (width 0.16) (layer "B.Cu") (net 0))
 (segment (start 128.006 98.064435) (end 128.960435 97.11) (width 0.16) (layer "B.Cu") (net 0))
 (segment (start 140.06 110.83) (end 140.06 110.3) (width 0.16) (layer "B.Cu") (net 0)))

